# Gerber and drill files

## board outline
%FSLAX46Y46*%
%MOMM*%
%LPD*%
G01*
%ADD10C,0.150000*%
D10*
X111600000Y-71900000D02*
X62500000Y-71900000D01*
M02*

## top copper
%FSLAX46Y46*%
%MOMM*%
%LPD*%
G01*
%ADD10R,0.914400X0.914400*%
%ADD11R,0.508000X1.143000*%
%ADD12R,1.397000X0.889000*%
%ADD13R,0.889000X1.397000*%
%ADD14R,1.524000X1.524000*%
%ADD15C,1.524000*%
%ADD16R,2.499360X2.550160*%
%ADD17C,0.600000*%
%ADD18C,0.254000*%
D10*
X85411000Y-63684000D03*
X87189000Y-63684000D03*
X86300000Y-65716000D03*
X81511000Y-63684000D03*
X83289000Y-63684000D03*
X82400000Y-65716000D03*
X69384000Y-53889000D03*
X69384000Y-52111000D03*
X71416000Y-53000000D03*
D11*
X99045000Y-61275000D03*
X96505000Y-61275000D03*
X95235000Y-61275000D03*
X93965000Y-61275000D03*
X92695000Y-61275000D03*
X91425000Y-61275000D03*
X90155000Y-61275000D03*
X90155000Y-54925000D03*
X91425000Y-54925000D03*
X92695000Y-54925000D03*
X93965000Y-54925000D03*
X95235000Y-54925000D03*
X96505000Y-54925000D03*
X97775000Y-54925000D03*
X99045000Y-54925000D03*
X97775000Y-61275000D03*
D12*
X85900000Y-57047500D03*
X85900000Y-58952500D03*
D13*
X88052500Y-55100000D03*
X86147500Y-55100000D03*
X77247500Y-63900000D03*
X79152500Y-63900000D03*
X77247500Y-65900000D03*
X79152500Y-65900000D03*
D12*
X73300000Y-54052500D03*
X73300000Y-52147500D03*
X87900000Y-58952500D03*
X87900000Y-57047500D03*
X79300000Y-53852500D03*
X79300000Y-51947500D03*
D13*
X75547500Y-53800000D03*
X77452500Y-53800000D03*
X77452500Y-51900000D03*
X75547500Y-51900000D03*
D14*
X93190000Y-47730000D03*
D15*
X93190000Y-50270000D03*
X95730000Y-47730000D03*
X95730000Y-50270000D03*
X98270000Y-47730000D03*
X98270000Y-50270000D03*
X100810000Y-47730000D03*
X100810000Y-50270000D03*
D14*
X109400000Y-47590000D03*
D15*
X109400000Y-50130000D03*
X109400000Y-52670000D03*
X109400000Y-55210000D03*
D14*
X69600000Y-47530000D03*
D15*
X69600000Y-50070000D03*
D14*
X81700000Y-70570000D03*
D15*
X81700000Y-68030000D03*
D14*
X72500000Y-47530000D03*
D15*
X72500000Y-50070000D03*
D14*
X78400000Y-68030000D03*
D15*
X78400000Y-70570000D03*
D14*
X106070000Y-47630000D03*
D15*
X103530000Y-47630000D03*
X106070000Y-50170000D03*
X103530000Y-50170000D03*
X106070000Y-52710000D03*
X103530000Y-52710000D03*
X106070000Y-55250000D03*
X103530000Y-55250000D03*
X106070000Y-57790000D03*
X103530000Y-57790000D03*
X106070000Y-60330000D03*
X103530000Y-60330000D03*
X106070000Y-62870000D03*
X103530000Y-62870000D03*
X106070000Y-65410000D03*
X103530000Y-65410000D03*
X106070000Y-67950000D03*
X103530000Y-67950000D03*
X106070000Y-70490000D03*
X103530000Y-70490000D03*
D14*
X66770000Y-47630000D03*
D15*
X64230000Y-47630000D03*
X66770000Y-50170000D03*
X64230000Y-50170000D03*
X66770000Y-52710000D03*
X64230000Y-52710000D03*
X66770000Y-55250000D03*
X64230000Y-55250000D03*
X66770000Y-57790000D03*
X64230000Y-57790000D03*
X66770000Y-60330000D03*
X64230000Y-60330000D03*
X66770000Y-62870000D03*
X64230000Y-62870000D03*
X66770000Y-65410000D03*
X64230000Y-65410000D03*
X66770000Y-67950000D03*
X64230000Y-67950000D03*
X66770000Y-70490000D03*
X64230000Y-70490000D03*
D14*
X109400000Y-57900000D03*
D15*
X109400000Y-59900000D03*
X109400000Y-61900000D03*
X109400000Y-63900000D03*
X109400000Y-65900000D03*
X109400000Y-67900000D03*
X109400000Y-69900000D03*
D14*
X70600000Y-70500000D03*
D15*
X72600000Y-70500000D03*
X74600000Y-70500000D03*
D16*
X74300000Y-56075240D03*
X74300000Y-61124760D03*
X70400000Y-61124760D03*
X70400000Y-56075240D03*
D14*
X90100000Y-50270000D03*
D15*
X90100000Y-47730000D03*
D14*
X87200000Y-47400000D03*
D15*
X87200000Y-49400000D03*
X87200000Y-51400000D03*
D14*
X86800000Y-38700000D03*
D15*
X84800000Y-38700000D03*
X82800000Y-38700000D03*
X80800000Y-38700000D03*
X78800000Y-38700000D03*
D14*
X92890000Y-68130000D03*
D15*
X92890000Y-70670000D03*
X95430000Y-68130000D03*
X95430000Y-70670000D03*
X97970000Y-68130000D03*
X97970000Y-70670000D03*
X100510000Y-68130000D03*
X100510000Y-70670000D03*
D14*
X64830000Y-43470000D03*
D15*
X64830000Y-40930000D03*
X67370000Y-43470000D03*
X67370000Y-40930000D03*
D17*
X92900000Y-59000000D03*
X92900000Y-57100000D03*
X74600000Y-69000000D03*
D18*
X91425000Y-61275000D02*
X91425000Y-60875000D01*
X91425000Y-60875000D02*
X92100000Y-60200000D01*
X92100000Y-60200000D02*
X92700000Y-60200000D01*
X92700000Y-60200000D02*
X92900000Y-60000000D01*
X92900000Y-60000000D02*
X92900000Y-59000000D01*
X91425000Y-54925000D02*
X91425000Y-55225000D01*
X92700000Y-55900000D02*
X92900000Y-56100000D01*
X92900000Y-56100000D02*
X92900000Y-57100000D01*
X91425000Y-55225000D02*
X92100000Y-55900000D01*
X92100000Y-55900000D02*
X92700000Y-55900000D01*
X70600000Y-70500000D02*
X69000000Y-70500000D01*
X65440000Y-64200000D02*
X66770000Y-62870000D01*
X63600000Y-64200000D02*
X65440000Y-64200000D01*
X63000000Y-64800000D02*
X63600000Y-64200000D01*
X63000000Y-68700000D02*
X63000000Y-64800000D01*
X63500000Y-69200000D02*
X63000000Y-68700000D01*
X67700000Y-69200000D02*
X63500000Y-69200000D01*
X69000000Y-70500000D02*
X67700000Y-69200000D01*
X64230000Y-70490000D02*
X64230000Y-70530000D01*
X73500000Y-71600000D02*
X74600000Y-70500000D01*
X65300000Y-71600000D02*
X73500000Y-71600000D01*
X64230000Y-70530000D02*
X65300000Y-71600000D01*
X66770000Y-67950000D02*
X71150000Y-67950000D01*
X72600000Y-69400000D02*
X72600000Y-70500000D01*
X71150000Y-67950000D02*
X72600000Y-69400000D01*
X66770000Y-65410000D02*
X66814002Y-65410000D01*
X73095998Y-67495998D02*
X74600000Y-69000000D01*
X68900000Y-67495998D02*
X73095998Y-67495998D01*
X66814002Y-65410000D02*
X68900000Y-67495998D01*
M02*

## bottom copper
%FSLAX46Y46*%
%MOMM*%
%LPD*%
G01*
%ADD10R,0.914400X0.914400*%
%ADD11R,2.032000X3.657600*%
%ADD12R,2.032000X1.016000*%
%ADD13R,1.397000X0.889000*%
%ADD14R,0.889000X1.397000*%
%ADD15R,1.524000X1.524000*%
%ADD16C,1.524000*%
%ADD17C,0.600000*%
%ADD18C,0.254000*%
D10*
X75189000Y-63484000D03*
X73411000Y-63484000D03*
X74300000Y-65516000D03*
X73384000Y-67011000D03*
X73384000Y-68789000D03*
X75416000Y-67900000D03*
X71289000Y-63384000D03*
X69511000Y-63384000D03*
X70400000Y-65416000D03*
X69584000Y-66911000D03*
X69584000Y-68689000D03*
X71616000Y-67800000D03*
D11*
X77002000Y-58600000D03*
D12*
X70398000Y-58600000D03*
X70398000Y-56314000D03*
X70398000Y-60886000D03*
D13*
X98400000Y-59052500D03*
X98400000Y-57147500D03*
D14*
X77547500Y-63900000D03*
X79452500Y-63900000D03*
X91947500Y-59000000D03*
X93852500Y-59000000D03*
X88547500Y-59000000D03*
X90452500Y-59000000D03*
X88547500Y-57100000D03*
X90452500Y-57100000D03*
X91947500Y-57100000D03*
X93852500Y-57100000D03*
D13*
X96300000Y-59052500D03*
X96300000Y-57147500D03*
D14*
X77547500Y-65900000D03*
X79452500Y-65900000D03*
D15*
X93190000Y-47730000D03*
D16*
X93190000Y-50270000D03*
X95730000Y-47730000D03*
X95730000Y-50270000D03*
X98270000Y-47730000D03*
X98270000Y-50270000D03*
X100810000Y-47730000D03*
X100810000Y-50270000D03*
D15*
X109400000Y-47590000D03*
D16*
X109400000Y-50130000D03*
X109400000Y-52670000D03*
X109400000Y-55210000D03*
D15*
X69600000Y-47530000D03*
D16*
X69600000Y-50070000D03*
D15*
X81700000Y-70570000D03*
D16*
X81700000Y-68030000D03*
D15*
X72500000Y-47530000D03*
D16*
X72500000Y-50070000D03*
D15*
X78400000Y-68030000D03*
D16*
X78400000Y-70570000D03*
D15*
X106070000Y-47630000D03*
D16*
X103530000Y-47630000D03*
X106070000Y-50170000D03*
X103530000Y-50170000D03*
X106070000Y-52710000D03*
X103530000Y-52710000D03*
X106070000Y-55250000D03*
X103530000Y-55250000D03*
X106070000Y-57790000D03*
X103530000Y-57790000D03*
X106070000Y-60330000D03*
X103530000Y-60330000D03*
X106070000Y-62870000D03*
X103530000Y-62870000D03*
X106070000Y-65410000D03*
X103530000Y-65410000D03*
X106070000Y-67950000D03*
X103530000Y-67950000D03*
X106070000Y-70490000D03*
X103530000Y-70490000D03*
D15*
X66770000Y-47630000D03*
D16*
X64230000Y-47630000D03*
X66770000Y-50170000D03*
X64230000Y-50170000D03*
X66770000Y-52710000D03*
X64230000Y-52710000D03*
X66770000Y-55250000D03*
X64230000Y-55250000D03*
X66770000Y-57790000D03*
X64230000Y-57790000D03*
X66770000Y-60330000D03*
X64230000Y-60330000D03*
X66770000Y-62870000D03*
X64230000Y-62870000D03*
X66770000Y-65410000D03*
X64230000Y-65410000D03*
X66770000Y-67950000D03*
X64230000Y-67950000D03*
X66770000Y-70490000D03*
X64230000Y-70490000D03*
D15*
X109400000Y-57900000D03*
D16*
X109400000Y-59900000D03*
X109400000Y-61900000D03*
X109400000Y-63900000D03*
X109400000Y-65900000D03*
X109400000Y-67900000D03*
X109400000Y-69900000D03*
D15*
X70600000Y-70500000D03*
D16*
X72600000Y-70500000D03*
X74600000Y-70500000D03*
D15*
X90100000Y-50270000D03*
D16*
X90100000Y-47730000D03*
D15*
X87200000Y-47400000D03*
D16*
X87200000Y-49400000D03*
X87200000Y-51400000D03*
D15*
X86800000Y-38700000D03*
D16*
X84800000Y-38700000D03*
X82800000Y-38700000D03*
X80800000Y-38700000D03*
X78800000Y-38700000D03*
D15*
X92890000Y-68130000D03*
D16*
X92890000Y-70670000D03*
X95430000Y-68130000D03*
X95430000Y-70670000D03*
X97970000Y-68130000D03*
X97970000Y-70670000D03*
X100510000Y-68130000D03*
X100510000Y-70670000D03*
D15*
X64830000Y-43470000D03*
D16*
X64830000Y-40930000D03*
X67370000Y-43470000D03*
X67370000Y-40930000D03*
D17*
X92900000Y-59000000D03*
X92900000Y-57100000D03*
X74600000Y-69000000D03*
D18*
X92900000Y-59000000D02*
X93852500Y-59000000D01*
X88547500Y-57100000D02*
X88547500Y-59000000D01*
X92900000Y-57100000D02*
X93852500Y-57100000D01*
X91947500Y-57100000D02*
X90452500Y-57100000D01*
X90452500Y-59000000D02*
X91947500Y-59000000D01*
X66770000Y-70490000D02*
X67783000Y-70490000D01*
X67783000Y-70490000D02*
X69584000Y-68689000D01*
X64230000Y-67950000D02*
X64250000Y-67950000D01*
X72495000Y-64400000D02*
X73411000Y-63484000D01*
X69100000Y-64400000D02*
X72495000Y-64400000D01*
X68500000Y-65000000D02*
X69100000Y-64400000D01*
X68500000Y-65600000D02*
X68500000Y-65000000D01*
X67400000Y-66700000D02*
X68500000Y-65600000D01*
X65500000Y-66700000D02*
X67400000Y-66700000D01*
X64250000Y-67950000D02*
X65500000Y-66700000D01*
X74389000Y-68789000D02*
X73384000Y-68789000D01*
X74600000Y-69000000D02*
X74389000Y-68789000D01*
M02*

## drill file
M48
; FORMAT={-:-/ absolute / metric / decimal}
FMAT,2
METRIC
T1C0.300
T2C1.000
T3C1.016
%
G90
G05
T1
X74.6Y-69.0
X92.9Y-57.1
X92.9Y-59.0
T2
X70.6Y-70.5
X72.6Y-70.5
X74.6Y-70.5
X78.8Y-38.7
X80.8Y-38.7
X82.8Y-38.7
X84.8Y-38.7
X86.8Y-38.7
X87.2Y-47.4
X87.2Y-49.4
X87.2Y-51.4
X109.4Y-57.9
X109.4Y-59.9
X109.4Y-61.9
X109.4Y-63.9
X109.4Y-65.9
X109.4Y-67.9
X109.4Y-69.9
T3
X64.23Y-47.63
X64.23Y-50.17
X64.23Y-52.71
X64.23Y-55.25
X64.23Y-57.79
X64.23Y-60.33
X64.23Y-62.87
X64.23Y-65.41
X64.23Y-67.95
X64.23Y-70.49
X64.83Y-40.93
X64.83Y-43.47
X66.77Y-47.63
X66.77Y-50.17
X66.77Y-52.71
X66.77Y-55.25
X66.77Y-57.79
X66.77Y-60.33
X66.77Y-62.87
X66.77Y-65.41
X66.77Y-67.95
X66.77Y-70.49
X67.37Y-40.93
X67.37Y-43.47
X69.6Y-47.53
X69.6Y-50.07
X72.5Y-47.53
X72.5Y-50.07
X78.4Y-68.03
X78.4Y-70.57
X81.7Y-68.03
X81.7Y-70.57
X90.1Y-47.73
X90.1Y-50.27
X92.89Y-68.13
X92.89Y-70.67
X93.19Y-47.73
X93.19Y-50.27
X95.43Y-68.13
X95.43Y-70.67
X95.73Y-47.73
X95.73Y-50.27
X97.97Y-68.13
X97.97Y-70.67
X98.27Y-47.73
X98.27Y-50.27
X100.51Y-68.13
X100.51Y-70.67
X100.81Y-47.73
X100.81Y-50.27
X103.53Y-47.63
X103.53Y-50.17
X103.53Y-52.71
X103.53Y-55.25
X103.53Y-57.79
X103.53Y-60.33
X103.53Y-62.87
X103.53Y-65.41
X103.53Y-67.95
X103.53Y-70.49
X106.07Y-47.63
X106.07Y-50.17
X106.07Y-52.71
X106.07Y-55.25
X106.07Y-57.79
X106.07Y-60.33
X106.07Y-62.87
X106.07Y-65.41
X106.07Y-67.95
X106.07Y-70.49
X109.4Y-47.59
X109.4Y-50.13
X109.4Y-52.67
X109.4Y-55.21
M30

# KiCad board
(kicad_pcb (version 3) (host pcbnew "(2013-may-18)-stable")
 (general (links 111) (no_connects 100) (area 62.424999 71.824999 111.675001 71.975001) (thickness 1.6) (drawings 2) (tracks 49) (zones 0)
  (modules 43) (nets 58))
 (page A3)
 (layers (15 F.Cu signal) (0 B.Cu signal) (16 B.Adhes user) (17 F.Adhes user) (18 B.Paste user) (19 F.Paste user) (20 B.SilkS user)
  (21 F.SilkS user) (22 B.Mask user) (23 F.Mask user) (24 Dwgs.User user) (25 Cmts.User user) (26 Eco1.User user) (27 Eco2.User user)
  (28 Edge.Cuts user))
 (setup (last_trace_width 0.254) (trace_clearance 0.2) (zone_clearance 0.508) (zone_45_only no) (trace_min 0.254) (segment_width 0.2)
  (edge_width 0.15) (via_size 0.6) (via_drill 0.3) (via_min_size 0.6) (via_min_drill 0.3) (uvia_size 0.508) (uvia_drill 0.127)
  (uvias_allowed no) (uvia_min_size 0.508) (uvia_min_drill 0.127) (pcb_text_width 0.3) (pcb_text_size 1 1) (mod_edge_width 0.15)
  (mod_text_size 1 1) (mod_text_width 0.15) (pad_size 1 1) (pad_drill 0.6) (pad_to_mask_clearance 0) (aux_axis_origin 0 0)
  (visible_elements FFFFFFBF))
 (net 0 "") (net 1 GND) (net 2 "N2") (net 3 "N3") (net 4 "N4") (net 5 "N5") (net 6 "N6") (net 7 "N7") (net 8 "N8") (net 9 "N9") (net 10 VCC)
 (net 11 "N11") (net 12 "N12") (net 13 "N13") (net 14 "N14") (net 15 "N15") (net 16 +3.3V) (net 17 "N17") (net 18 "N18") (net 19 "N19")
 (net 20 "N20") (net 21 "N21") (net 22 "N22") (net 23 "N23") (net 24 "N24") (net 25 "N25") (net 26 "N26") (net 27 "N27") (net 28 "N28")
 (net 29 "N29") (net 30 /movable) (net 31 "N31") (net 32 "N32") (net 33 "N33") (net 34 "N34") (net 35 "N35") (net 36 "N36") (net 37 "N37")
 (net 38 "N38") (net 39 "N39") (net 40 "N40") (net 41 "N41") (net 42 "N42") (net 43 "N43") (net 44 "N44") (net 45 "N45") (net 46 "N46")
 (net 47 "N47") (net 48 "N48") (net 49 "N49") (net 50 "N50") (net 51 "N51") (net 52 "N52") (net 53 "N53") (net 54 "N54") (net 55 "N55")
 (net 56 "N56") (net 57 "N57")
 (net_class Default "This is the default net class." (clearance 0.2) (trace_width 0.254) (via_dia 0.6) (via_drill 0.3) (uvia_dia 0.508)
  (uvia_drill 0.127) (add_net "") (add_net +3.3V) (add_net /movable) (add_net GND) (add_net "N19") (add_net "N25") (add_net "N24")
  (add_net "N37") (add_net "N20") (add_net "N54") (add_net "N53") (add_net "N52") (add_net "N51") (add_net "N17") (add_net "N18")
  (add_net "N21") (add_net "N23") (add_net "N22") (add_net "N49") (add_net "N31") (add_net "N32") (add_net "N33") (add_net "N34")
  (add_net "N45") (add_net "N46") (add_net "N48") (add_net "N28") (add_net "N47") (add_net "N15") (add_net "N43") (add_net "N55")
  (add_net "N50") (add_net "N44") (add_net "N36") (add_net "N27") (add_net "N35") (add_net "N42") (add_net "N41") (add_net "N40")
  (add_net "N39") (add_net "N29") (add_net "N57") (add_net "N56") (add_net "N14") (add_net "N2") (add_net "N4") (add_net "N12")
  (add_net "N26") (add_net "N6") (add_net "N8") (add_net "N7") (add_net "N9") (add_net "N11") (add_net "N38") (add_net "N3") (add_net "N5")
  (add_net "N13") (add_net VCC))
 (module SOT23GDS (layer B.Cu) (at 74.3 64.5 180)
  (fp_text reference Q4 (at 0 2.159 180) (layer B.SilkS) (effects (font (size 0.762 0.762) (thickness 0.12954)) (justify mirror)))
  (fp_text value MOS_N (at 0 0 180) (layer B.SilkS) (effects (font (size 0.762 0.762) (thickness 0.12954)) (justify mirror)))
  (pad S smd rect (at -0.889 1.016 180) (size 0.9144 0.9144) (layers B.Cu B.Paste B.Mask) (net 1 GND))
  (pad G smd rect (at 0.889 1.016 180) (size 0.9144 0.9144) (layers B.Cu B.Paste B.Mask) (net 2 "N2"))
  (pad D smd rect (at 0 -1.016 180) (size 0.9144 0.9144) (layers B.Cu B.Paste B.Mask) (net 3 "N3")))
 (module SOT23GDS (layer B.Cu) (at 74.4 67.9 270)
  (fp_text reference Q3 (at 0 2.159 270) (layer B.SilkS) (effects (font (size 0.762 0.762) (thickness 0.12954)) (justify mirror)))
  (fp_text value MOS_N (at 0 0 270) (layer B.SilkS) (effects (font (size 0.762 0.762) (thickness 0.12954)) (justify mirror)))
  (pad S smd rect (at -0.889 1.016 270) (size 0.9144 0.9144) (layers B.Cu B.Paste B.Mask) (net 1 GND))
  (pad G smd rect (at 0.889 1.016 270) (size 0.9144 0.9144) (layers B.Cu B.Paste B.Mask) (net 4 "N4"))
  (pad D smd rect (at 0 -1.016 270) (size 0.9144 0.9144) (layers B.Cu B.Paste B.Mask) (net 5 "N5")))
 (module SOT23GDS (layer F.Cu) (at 86.3 64.7)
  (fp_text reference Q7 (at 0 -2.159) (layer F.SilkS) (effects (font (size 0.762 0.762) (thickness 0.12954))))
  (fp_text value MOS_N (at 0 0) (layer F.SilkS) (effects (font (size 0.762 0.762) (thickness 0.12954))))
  (pad S smd rect (at -0.889 -1.016) (size 0.9144 0.9144) (layers F.Cu F.Paste F.Mask) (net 1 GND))
  (pad G smd rect (at 0.889 -1.016) (size 0.9144 0.9144) (layers F.Cu F.Paste F.Mask) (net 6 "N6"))
  (pad D smd rect (at 0 1.016) (size 0.9144 0.9144) (layers F.Cu F.Paste F.Mask) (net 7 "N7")))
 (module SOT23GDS (layer F.Cu) (at 82.4 64.7)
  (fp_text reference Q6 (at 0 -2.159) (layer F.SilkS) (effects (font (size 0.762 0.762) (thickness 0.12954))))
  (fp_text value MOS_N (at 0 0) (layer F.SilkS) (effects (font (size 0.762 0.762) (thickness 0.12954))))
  (pad S smd rect (at -0.889 -1.016) (size 0.9144 0.9144) (layers F.Cu F.Paste F.Mask) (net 1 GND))
  (pad G smd rect (at 0.889 -1.016) (size 0.9144 0.9144) (layers F.Cu F.Paste F.Mask) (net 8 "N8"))
  (pad D smd rect (at 0 1.016) (size 0.9144 0.9144) (layers F.Cu F.Paste F.Mask) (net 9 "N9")))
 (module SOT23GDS (layer F.Cu) (at 70.4 53 90)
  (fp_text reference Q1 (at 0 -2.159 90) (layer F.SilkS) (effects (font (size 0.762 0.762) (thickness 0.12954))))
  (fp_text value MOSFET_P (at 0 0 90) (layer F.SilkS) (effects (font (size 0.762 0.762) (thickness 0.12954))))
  (pad S smd rect (at -0.889 -1.016 90) (size 0.9144 0.9144) (layers F.Cu F.Paste F.Mask) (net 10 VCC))
  (pad G smd rect (at 0.889 -1.016 90) (size 0.9144 0.9144) (layers F.Cu F.Paste F.Mask) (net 1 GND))
  (pad D smd rect (at 0 1.016 90) (size 0.9144 0.9144) (layers F.Cu F.Paste F.Mask) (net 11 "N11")))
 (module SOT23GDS (layer B.Cu) (at 70.4 64.4 180)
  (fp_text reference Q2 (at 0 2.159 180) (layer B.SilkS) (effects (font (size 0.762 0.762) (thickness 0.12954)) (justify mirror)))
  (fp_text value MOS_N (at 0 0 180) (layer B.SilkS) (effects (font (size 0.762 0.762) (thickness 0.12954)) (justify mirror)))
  (pad S smd rect (at -0.889 1.016 180) (size 0.9144 0.9144) (layers B.Cu B.Paste B.Mask) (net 1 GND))
  (pad G smd rect (at 0.889 1.016 180) (size 0.9144 0.9144) (layers B.Cu B.Paste B.Mask) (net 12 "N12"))
  (pad D smd rect (at 0 -1.016 180) (size 0.9144 0.9144) (layers B.Cu B.Paste B.Mask) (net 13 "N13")))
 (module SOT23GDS (layer B.Cu) (at 70.6 67.8 270)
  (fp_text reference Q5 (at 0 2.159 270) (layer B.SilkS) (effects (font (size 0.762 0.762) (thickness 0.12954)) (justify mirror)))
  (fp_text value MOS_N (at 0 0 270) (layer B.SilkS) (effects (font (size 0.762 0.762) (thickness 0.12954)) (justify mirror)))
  (pad S smd rect (at -0.889 1.016 270) (size 0.9144 0.9144) (layers B.Cu B.Paste B.Mask) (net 1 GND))
  (pad G smd rect (at 0.889 1.016 270) (size 0.9144 0.9144) (layers B.Cu B.Paste B.Mask) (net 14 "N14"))
  (pad D smd rect (at 0 -1.016 270) (size 0.9144 0.9144) (layers B.Cu B.Paste B.Mask) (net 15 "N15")))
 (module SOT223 (layer B.Cu) (at 73.7 58.6 90)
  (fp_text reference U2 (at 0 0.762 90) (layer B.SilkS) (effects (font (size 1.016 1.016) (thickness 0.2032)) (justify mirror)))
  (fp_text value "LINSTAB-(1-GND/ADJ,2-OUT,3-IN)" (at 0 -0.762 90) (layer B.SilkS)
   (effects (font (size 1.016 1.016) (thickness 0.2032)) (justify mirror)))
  (pad 4 smd rect (at 0 3.302 90) (size 3.6576 2.032) (layers B.Cu B.Paste B.Mask))
  (pad 2 smd rect (at 0 -3.302 90) (size 1.016 2.032) (layers B.Cu B.Paste B.Mask) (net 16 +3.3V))
  (pad 3 smd rect (at 2.286 -3.302 90) (size 1.016 2.032) (layers B.Cu B.Paste B.Mask) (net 10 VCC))
  (pad 1 smd rect (at -2.286 -3.302 90) (size 1.016 2.032) (layers B.Cu B.Paste B.Mask) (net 1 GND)))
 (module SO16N (layer F.Cu) (at 94.6 58.1 180)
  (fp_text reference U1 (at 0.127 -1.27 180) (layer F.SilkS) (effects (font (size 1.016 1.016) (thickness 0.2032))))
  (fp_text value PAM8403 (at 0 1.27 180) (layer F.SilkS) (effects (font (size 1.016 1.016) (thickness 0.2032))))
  (pad 16 smd rect (at -4.445 -3.175 180) (size 0.508 1.143) (layers F.Cu F.Paste F.Mask) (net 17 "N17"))
  (pad 14 smd rect (at -1.905 -3.175 180) (size 0.508 1.143) (layers F.Cu F.Paste F.Mask) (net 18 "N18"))
  (pad 13 smd rect (at -0.635 -3.175 180) (size 0.508 1.143) (layers F.Cu F.Paste F.Mask) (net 10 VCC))
  (pad 12 smd rect (at 0.635 -3.175 180) (size 0.508 1.143) (layers F.Cu F.Paste F.Mask) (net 10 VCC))
  (pad 11 smd rect (at 1.905 -3.175 180) (size 0.508 1.143) (layers F.Cu F.Paste F.Mask) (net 1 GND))
  (pad 10 smd rect (at 3.175 -3.175 180) (size 0.508 1.143) (layers F.Cu F.Paste F.Mask) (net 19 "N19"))
  (pad 9 smd rect (at 4.445 -3.175 180) (size 0.508 1.143) (layers F.Cu F.Paste F.Mask) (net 1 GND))
  (pad 8 smd rect (at 4.445 3.175 180) (size 0.508 1.143) (layers F.Cu F.Paste F.Mask) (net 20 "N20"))
  (pad 7 smd rect (at 3.175 3.175 180) (size 0.508 1.143) (layers F.Cu F.Paste F.Mask) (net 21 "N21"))
  (pad 6 smd rect (at 1.905 3.175 180) (size 0.508 1.143) (layers F.Cu F.Paste F.Mask) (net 10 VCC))
  (pad 5 smd rect (at 0.635 3.175 180) (size 0.508 1.143) (layers F.Cu F.Paste F.Mask) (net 10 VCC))
  (pad 4 smd rect (at -0.635 3.175 180) (size 0.508 1.143) (layers F.Cu F.Paste F.Mask) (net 10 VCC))
  (pad 3 smd rect (at -1.905 3.175 180) (size 0.508 1.143) (layers F.Cu F.Paste F.Mask) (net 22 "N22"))
  (pad 2 smd rect (at -3.175 3.175 180) (size 0.508 1.143) (layers F.Cu F.Paste F.Mask) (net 1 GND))
  (pad 1 smd rect (at -4.445 3.175 180) (size 0.508 1.143) (layers F.Cu F.Paste F.Mask) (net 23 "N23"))
  (pad 15 smd rect (at -3.175 -3.175 180) (size 0.508 1.143) (layers F.Cu F.Paste F.Mask) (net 1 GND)))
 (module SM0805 (layer B.Cu) (at 98.4 58.1 90)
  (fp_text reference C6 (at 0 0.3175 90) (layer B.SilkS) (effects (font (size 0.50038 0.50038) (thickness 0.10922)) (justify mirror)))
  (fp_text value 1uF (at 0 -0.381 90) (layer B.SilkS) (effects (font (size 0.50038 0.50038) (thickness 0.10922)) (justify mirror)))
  (pad 1 smd rect (at -0.9525 0 90) (size 0.889 1.397) (layers B.Cu B.Paste B.Mask) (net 10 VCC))
  (pad 2 smd rect (at 0.9525 0 90) (size 0.889 1.397) (layers B.Cu B.Paste B.Mask) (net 1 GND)))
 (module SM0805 (layer F.Cu) (at 85.9 58 270)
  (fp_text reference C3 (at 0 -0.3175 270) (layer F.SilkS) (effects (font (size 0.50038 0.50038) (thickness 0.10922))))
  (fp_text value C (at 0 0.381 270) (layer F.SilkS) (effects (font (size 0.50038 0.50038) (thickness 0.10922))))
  (pad 1 smd rect (at -0.9525 0 270) (size 0.889 1.397) (layers F.Cu F.Paste F.Mask) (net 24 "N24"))
  (pad 2 smd rect (at 0.9525 0 270) (size 0.889 1.397) (layers F.Cu F.Paste F.Mask) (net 1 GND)))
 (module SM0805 (layer F.Cu) (at 87.1 55.1 180)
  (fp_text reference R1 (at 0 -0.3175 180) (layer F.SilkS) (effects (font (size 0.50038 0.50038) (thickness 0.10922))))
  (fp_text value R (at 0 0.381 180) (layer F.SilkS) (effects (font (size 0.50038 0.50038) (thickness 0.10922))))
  (pad 1 smd rect (at -0.9525 0 180) (size 0.889 1.397) (layers F.Cu F.Paste F.Mask) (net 24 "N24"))
  (pad 2 smd rect (at 0.9525 0 180) (size 0.889 1.397) (layers F.Cu F.Paste F.Mask) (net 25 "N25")))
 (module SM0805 (layer F.Cu) (at 78.2 63.9)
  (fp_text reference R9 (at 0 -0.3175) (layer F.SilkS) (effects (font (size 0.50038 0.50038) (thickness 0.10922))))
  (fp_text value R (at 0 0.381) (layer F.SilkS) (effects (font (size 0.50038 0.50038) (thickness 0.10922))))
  (pad 1 smd rect (at -0.9525 0) (size 0.889 1.397) (layers F.Cu F.Paste F.Mask) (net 15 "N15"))
  (pad 2 smd rect (at 0.9525 0) (size 0.889 1.397) (layers F.Cu F.Paste F.Mask) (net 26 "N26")))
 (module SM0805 (layer B.Cu) (at 78.5 63.9)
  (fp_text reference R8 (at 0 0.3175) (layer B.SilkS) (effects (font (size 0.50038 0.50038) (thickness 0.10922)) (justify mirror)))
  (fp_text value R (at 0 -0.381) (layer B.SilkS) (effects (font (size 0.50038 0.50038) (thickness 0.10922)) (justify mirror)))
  (pad 1 smd rect (at -0.9525 0) (size 0.889 1.397) (layers B.Cu B.Paste B.Mask) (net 3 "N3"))
  (pad 2 smd rect (at 0.9525 0) (size 0.889 1.397) (layers B.Cu B.Paste B.Mask) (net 26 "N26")))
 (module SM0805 (layer F.Cu) (at 78.2 65.9)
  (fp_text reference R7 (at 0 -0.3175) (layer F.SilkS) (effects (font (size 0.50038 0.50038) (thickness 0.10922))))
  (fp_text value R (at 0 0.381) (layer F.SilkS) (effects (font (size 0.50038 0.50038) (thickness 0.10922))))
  (pad 1 smd rect (at -0.9525 0) (size 0.889 1.397) (layers F.Cu F.Paste F.Mask) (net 5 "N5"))
  (pad 2 smd rect (at 0.9525 0) (size 0.889 1.397) (layers F.Cu F.Paste F.Mask) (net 26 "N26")))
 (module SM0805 (layer B.Cu) (at 92.9 59)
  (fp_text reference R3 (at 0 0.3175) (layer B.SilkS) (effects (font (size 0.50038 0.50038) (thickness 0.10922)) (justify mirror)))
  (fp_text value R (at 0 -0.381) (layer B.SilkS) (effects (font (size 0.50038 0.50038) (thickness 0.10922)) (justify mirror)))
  (pad 1 smd rect (at -0.9525 0) (size 0.889 1.397) (layers B.Cu B.Paste B.Mask) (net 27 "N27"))
  (pad 2 smd rect (at 0.9525 0) (size 0.889 1.397) (layers B.Cu B.Paste B.Mask) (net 19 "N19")))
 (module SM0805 (layer B.Cu) (at 89.5 59)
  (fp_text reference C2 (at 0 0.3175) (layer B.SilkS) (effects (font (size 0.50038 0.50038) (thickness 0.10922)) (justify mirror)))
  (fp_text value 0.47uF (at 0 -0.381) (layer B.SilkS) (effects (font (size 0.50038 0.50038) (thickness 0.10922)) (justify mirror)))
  (pad 1 smd rect (at -0.9525 0) (size 0.889 1.397) (layers B.Cu B.Paste B.Mask) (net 24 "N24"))
  (pad 2 smd rect (at 0.9525 0) (size 0.889 1.397) (layers B.Cu B.Paste B.Mask) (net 27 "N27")))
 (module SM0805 (layer B.Cu) (at 89.5 57.1)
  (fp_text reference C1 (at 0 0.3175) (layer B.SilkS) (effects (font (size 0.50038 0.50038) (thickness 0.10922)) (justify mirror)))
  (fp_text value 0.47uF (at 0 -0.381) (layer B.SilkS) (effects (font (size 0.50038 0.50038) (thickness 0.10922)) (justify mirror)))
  (pad 1 smd rect (at -0.9525 0) (size 0.889 1.397) (layers B.Cu B.Paste B.Mask) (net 24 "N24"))
  (pad 2 smd rect (at 0.9525 0) (size 0.889 1.397) (layers B.Cu B.Paste B.Mask) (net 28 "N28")))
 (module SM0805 (layer B.Cu) (at 92.9 57.1)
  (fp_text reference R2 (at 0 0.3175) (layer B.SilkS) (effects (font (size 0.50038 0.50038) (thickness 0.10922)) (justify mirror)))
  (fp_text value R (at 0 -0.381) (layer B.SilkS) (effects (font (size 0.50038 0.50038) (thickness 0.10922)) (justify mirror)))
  (pad 1 smd rect (at -0.9525 0) (size 0.889 1.397) (layers B.Cu B.Paste B.Mask) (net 28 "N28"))
  (pad 2 smd rect (at 0.9525 0) (size 0.889 1.397) (layers B.Cu B.Paste B.Mask) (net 21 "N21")))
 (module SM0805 (layer F.Cu) (at 73.3 53.1 90)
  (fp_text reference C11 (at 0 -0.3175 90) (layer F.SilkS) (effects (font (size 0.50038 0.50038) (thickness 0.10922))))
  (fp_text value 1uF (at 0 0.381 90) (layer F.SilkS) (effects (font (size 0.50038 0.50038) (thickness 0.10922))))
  (pad 1 smd rect (at -0.9525 0 90) (size 0.889 1.397) (layers F.Cu F.Paste F.Mask) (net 10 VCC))
  (pad 2 smd rect (at 0.9525 0 90) (size 0.889 1.397) (layers F.Cu F.Paste F.Mask) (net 1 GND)))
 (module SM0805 (layer B.Cu) (at 96.3 58.1 90)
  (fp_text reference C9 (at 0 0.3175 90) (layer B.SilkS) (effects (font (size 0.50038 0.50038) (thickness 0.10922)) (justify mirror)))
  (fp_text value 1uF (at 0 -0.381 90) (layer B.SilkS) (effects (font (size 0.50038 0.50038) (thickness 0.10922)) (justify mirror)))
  (pad 1 smd rect (at -0.9525 0 90) (size 0.889 1.397) (layers B.Cu B.Paste B.Mask) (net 10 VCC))
  (pad 2 smd rect (at 0.9525 0 90) (size 0.889 1.397) (layers B.Cu B.Paste B.Mask) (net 1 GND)))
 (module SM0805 (layer B.Cu) (at 78.5 65.9)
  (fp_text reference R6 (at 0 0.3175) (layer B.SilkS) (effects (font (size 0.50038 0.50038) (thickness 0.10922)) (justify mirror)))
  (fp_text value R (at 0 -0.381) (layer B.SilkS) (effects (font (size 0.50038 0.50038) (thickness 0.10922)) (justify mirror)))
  (pad 1 smd rect (at -0.9525 0) (size 0.889 1.397) (layers B.Cu B.Paste B.Mask) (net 13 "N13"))
  (pad 2 smd rect (at 0.9525 0) (size 0.889 1.397) (layers B.Cu B.Paste B.Mask) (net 26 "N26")))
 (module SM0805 (layer F.Cu) (at 87.9 58 90)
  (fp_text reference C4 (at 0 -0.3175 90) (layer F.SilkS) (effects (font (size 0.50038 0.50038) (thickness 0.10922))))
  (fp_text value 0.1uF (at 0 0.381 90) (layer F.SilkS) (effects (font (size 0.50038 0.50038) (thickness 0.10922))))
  (pad 1 smd rect (at -0.9525 0 90) (size 0.889 1.397) (layers F.Cu F.Paste F.Mask) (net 1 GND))
  (pad 2 smd rect (at 0.9525 0 90) (size 0.889 1.397) (layers F.Cu F.Paste F.Mask) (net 20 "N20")))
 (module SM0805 (layer F.Cu) (at 79.3 52.9 90)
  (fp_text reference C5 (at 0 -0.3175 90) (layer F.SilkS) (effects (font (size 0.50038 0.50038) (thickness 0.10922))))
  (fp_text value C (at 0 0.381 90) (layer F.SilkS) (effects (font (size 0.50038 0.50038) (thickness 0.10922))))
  (pad 1 smd rect (at -0.9525 0 90) (size 0.889 1.397) (layers F.Cu F.Paste F.Mask) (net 10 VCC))
  (pad 2 smd rect (at 0.9525 0 90) (size 0.889 1.397) (layers F.Cu F.Paste F.Mask) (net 1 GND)))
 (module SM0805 (layer F.Cu) (at 76.5 53.8)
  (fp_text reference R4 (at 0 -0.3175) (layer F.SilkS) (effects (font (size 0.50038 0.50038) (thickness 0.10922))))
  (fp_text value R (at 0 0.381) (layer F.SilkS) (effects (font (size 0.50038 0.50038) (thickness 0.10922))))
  (pad 1 smd rect (at -0.9525 0) (size 0.889 1.397) (layers F.Cu F.Paste F.Mask) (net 10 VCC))
  (pad 2 smd rect (at 0.9525 0) (size 0.889 1.397) (layers F.Cu F.Paste F.Mask) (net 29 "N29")))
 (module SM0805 (layer F.Cu) (at 76.5 51.9 180)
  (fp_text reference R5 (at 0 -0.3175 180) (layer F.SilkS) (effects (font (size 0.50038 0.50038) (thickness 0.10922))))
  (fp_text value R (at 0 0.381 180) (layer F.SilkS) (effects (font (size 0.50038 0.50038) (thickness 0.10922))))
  (pad 1 smd rect (at -0.9525 0 180) (size 0.889 1.397) (layers F.Cu F.Paste F.Mask) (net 29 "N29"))
  (pad 2 smd rect (at 0.9525 0 180) (size 0.889 1.397) (layers F.Cu F.Paste F.Mask) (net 1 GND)))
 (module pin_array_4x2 (layer B.Cu) (at 97 49)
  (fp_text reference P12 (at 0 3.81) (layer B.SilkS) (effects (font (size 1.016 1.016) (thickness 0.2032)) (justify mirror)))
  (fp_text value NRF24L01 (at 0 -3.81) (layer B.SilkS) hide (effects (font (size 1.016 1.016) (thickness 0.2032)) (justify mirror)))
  (pad 1 thru_hole rect (at -3.81 -1.27) (size 1.524 1.524) (drill 1.016) (layers *.Cu *.Mask B.SilkS) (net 1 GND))
  (pad 2 thru_hole circle (at -3.81 1.27) (size 1.524 1.524) (drill 1.016) (layers *.Cu *.Mask B.SilkS) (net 16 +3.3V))
  (pad 3 thru_hole circle (at -1.27 -1.27) (size 1.524 1.524) (drill 1.016) (layers *.Cu *.Mask B.SilkS) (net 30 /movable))
  (pad 4 thru_hole circle (at -1.27 1.27) (size 1.524 1.524) (drill 1.016) (layers *.Cu *.Mask B.SilkS) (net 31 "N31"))
  (pad 5 thru_hole circle (at 1.27 -1.27) (size 1.524 1.524) (drill 1.016) (layers *.Cu *.Mask B.SilkS) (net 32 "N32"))
  (pad 6 thru_hole circle (at 1.27 1.27) (size 1.524 1.524) (drill 1.016) (layers *.Cu *.Mask B.SilkS) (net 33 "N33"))
  (pad 7 thru_hole circle (at 3.81 -1.27) (size 1.524 1.524) (drill 1.016) (layers *.Cu *.Mask B.SilkS) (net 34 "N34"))
  (pad 8 thru_hole circle (at 3.81 1.27) (size 1.524 1.524) (drill 1.016) (layers *.Cu *.Mask B.SilkS) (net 30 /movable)))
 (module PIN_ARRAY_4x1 (layer B.Cu) (at 109.4 51.4 270)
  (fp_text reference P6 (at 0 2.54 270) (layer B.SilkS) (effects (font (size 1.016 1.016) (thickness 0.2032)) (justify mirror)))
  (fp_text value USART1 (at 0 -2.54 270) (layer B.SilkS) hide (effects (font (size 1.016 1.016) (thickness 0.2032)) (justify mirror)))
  (pad 1 thru_hole rect (at -3.81 0 270) (size 1.524 1.524) (drill 1.016) (layers *.Cu *.Mask B.SilkS) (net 1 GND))
  (pad 2 thru_hole circle (at -1.27 0 270) (size 1.524 1.524) (drill 1.016) (layers *.Cu *.Mask B.SilkS))
  (pad 3 thru_hole circle (at 1.27 0 270) (size 1.524 1.524) (drill 1.016) (layers *.Cu *.Mask B.SilkS) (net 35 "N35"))
  (pad 4 thru_hole circle (at 3.81 0 270) (size 1.524 1.524) (drill 1.016) (layers *.Cu *.Mask B.SilkS) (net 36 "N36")))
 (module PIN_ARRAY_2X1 (layer B.Cu) (at 69.6 48.8 270)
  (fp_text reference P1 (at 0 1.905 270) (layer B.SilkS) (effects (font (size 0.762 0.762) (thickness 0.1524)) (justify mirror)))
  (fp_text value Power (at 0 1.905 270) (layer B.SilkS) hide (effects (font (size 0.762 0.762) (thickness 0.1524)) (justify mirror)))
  (pad 1 thru_hole rect (at -1.27 0 270) (size 1.524 1.524) (drill 1.016) (layers *.Cu *.Mask B.SilkS) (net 1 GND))
  (pad 2 thru_hole circle (at 1.27 0 270) (size 1.524 1.524) (drill 1.016) (layers *.Cu *.Mask B.SilkS) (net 11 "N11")))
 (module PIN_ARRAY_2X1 (layer B.Cu) (at 81.7 69.3 90)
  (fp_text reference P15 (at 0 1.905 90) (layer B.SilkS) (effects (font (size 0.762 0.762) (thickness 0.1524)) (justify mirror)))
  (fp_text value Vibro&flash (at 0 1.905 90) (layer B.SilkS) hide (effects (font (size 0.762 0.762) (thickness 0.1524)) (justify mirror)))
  (pad 1 thru_hole rect (at -1.27 0 90) (size 1.524 1.524) (drill 1.016) (layers *.Cu *.Mask B.SilkS) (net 7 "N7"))
  (pad 2 thru_hole circle (at 1.27 0 90) (size 1.524 1.524) (drill 1.016) (layers *.Cu *.Mask B.SilkS) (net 9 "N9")))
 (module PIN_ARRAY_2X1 (layer B.Cu) (at 72.5 48.8 270)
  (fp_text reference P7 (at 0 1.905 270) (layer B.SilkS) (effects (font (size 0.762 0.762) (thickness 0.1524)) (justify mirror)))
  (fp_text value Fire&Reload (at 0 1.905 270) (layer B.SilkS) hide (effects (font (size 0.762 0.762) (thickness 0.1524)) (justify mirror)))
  (pad 1 thru_hole rect (at -1.27 0 270) (size 1.524 1.524) (drill 1.016) (layers *.Cu *.Mask B.SilkS) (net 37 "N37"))
  (pad 2 thru_hole circle (at 1.27 0 270) (size 1.524 1.524) (drill 1.016) (layers *.Cu *.Mask B.SilkS) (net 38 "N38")))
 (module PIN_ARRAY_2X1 (layer B.Cu) (at 78.4 69.3 270)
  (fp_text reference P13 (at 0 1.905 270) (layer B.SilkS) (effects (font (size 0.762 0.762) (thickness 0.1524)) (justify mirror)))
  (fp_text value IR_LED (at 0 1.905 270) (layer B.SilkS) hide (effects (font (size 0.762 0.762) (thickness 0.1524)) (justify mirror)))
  (pad 1 thru_hole rect (at -1.27 0 270) (size 1.524 1.524) (drill 1.016) (layers *.Cu *.Mask B.SilkS) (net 26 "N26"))
  (pad 2 thru_hole circle (at 1.27 0 270) (size 1.524 1.524) (drill 1.016) (layers *.Cu *.Mask B.SilkS) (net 10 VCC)))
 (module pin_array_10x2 (layer B.Cu) (at 104.8 59.1 270)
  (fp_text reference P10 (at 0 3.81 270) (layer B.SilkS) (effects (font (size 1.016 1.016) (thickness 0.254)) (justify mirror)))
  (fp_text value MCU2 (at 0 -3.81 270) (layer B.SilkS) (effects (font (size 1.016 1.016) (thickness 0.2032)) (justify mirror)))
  (pad 1 thru_hole rect (at -11.47 -1.27 270) (size 1.524 1.524) (drill 1.016) (layers *.Cu *.Mask B.SilkS) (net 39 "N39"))
  (pad 2 thru_hole circle (at -11.47 1.27 270) (size 1.524 1.524) (drill 1.016) (layers *.Cu *.Mask B.SilkS) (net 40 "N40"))
  (pad 3 thru_hole circle (at -8.93 -1.27 270) (size 1.524 1.524) (drill 1.016) (layers *.Cu *.Mask B.SilkS) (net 31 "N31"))
  (pad 4 thru_hole circle (at -8.93 1.27 270) (size 1.524 1.524) (drill 1.016) (layers *.Cu *.Mask B.SilkS) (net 32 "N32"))
  (pad 5 thru_hole circle (at -6.39 -1.27 270) (size 1.524 1.524) (drill 1.016) (layers *.Cu *.Mask B.SilkS) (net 34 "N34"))
  (pad 6 thru_hole circle (at -6.39 1.27 270) (size 1.524 1.524) (drill 1.016) (layers *.Cu *.Mask B.SilkS) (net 33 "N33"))
  (pad 7 thru_hole circle (at -3.85 -1.27 270) (size 1.524 1.524) (drill 1.016) (layers *.Cu *.Mask B.SilkS) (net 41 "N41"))
  (pad 8 thru_hole circle (at -3.85 1.27 270) (size 1.524 1.524) (drill 1.016) (layers *.Cu *.Mask B.SilkS) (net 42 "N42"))
  (pad 9 thru_hole circle (at -1.31 -1.27 270) (size 1.524 1.524) (drill 1.016) (layers *.Cu *.Mask B.SilkS) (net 35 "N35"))
  (pad 10 thru_hole circle (at -1.31 1.27 270) (size 1.524 1.524) (drill 1.016) (layers *.Cu *.Mask B.SilkS) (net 36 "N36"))
  (pad 11 thru_hole circle (at 1.23 -1.27 270) (size 1.524 1.524) (drill 1.016) (layers *.Cu *.Mask B.SilkS) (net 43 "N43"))
  (pad 12 thru_hole circle (at 1.23 1.27 270) (size 1.524 1.524) (drill 1.016) (layers *.Cu *.Mask B.SilkS) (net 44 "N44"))
  (pad 13 thru_hole circle (at 3.77 -1.27 270) (size 1.524 1.524) (drill 1.016) (layers *.Cu *.Mask B.SilkS) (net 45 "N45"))
  (pad 14 thru_hole circle (at 3.77 1.27 270) (size 1.524 1.524) (drill 1.016) (layers *.Cu *.Mask B.SilkS) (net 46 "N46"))
  (pad 15 thru_hole circle (at 6.31 -1.27 270) (size 1.524 1.524) (drill 1.016) (layers *.Cu *.Mask B.SilkS) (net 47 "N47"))
  (pad 16 thru_hole circle (at 6.31 1.27 270) (size 1.524 1.524) (drill 1.016) (layers *.Cu *.Mask B.SilkS) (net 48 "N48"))
  (pad 17 thru_hole circle (at 8.85 -1.27 270) (size 1.524 1.524) (drill 1.016) (layers *.Cu *.Mask B.SilkS) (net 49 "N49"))
  (pad 18 thru_hole circle (at 8.85 1.27 270) (size 1.524 1.524) (drill 1.016) (layers *.Cu *.Mask B.SilkS) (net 30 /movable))
  (pad 19 thru_hole circle (at 11.39 -1.27 270) (size 1.524 1.524) (drill 1.016) (layers *.Cu *.Mask B.SilkS) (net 30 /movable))
  (pad 20 thru_hole circle (at 11.39 1.27 270) (size 1.524 1.524) (drill 1.016) (layers *.Cu *.Mask B.SilkS) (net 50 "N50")))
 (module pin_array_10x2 (layer B.Cu) (at 65.5 59.1 270)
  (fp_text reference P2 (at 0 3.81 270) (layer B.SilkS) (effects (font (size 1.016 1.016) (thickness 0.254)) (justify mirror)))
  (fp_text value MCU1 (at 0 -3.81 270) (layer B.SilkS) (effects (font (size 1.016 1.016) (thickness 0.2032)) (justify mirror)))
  (pad 1 thru_hole rect (at -11.47 -1.27 270) (size 1.524 1.524) (drill 1.016) (layers *.Cu *.Mask B.SilkS) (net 1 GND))
  (pad 2 thru_hole circle (at -11.47 1.27 270) (size 1.524 1.524) (drill 1.016) (layers *.Cu *.Mask B.SilkS) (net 16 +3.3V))
  (pad 3 thru_hole circle (at -8.93 -1.27 270) (size 1.524 1.524) (drill 1.016) (layers *.Cu *.Mask B.SilkS))
  (pad 4 thru_hole circle (at -8.93 1.27 270) (size 1.524 1.524) (drill 1.016) (layers *.Cu *.Mask B.SilkS) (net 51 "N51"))
  (pad 5 thru_hole circle (at -6.39 -1.27 270) (size 1.524 1.524) (drill 1.016) (layers *.Cu *.Mask B.SilkS) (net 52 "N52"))
  (pad 6 thru_hole circle (at -6.39 1.27 270) (size 1.524 1.524) (drill 1.016) (layers *.Cu *.Mask B.SilkS) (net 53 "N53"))
  (pad 7 thru_hole circle (at -3.85 -1.27 270) (size 1.524 1.524) (drill 1.016) (layers *.Cu *.Mask B.SilkS) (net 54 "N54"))
  (pad 8 thru_hole circle (at -3.85 1.27 270) (size 1.524 1.524) (drill 1.016) (layers *.Cu *.Mask B.SilkS) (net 37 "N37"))
  (pad 9 thru_hole circle (at -1.31 -1.27 270) (size 1.524 1.524) (drill 1.016) (layers *.Cu *.Mask B.SilkS) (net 38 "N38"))
  (pad 10 thru_hole circle (at -1.31 1.27 270) (size 1.524 1.524) (drill 1.016) (layers *.Cu *.Mask B.SilkS) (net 8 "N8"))
  (pad 11 thru_hole circle (at 1.23 -1.27 270) (size 1.524 1.524) (drill 1.016) (layers *.Cu *.Mask B.SilkS) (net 6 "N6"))
  (pad 12 thru_hole circle (at 1.23 1.27 270) (size 1.524 1.524) (drill 1.016) (layers *.Cu *.Mask B.SilkS) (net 25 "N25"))
  (pad 13 thru_hole circle (at 3.77 -1.27 270) (size 1.524 1.524) (drill 1.016) (layers *.Cu *.Mask B.SilkS) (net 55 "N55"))
  (pad 14 thru_hole circle (at 3.77 1.27 270) (size 1.524 1.524) (drill 1.016) (layers *.Cu *.Mask B.SilkS) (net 12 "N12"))
  (pad 15 thru_hole circle (at 6.31 -1.27 270) (size 1.524 1.524) (drill 1.016) (layers *.Cu *.Mask B.SilkS) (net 4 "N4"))
  (pad 16 thru_hole circle (at 6.31 1.27 270) (size 1.524 1.524) (drill 1.016) (layers *.Cu *.Mask B.SilkS) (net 29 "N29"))
  (pad 17 thru_hole circle (at 8.85 -1.27 270) (size 1.524 1.524) (drill 1.016) (layers *.Cu *.Mask B.SilkS) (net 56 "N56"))
  (pad 18 thru_hole circle (at 8.85 1.27 270) (size 1.524 1.524) (drill 1.016) (layers *.Cu *.Mask B.SilkS) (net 2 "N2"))
  (pad 19 thru_hole circle (at 11.39 -1.27 270) (size 1.524 1.524) (drill 1.016) (layers *.Cu *.Mask B.SilkS) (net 14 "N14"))
  (pad 20 thru_hole circle (at 11.39 1.27 270) (size 1.524 1.524) (drill 1.016) (layers *.Cu *.Mask B.SilkS) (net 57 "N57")))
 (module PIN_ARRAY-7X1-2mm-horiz (layer F.Cu) (at 109.4 63.9 270)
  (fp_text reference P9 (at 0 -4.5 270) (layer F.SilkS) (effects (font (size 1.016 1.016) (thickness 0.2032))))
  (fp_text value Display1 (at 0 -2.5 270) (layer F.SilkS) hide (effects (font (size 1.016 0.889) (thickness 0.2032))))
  (pad 1 thru_hole rect (at -6 0 270) (size 1.524 1.524) (drill 1) (layers *.Cu *.Mask F.SilkS) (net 39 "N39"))
  (pad 2 thru_hole circle (at -4 0 270) (size 1.524 1.524) (drill 1) (layers *.Cu *.Mask F.SilkS) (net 40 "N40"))
  (pad 3 thru_hole circle (at -2 0 270) (size 1.524 1.524) (drill 1) (layers *.Cu *.Mask F.SilkS) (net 41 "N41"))
  (pad 4 thru_hole circle (at 0 0 270) (size 1.524 1.524) (drill 1) (layers *.Cu *.Mask F.SilkS) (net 42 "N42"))
  (pad 5 thru_hole circle (at 2 0 270) (size 1.524 1.524) (drill 1) (layers *.Cu *.Mask F.SilkS) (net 43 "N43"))
  (pad 6 thru_hole circle (at 4 0 270) (size 1.524 1.524) (drill 1) (layers *.Cu *.Mask F.SilkS) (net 44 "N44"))
  (pad 7 thru_hole circle (at 6 0 270) (size 1.524 1.524) (drill 1) (layers *.Cu *.Mask F.SilkS) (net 50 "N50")))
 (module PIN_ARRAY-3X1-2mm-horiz (layer B.Cu) (at 72.6 70.5)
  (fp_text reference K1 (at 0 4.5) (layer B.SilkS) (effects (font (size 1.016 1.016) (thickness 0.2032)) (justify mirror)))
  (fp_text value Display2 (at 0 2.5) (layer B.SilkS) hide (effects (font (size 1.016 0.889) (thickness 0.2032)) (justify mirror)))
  (pad 1 thru_hole rect (at -2 0) (size 1.524 1.524) (drill 1) (layers *.Cu *.Mask B.SilkS) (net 55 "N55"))
  (pad 2 thru_hole circle (at 0 0) (size 1.524 1.524) (drill 1) (layers *.Cu *.Mask B.SilkS) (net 56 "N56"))
  (pad 3 thru_hole circle (at 2 0) (size 1.524 1.524) (drill 1) (layers *.Cu *.Mask B.SilkS) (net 57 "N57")))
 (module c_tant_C (layer F.Cu) (at 74.3 58.6 90)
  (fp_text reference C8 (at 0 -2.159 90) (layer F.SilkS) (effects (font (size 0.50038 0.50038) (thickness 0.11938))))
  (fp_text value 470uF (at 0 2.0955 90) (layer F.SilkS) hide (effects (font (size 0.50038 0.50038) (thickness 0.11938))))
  (pad 1 smd rect (at 2.52476 0 90) (size 2.55016 2.49936) (layers F.Cu F.Paste F.Mask) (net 10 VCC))
  (pad 2 smd rect (at -2.52476 0 90) (size 2.55016 2.49936) (layers F.Cu F.Paste F.Mask) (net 1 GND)))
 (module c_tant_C (layer F.Cu) (at 70.4 58.6 270)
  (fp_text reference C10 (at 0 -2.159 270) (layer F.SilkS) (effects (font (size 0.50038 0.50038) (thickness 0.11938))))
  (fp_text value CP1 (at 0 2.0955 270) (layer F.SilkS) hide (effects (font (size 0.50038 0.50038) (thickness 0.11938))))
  (pad 1 smd rect (at 2.52476 0 270) (size 2.55016 2.49936) (layers F.Cu F.Paste F.Mask) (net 16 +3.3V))
  (pad 2 smd rect (at -2.52476 0 270) (size 2.55016 2.49936) (layers F.Cu F.Paste F.Mask) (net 1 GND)))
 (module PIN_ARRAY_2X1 (layer B.Cu) (at 90.1 49 90)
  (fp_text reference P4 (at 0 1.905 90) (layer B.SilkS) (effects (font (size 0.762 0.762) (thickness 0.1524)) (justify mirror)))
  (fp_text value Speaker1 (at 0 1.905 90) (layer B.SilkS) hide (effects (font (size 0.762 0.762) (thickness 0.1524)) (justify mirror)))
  (pad 1 thru_hole rect (at -1.27 0 90) (size 1.524 1.524) (drill 1.016) (layers *.Cu *.Mask B.SilkS) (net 22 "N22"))
  (pad 2 thru_hole circle (at 1.27 0 90) (size 1.524 1.524) (drill 1.016) (layers *.Cu *.Mask B.SilkS) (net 23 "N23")))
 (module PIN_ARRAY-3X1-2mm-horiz (layer B.Cu) (at 87.2 49.4 270)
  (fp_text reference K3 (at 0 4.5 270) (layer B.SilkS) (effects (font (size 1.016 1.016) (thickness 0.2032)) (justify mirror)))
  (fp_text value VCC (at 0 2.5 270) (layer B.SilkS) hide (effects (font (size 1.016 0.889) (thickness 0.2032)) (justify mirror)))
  (pad 1 thru_hole rect (at -2 0 270) (size 1.524 1.524) (drill 1) (layers *.Cu *.Mask B.SilkS) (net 10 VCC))
  (pad 2 thru_hole circle (at 0 0 270) (size 1.524 1.524) (drill 1) (layers *.Cu *.Mask B.SilkS) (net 10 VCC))
  (pad 3 thru_hole circle (at 2 0 270) (size 1.524 1.524) (drill 1) (layers *.Cu *.Mask B.SilkS) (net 10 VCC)))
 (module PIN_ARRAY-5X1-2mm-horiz (layer B.Cu) (at 82.8 38.7 180)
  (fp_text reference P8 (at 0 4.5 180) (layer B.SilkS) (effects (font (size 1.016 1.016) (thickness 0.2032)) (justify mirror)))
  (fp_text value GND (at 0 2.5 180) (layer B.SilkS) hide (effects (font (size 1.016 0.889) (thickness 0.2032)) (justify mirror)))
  (pad 1 thru_hole rect (at -4 0 180) (size 1.524 1.524) (drill 1) (layers *.Cu *.Mask B.SilkS) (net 1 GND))
  (pad 2 thru_hole circle (at -2 0 180) (size 1.524 1.524) (drill 1) (layers *.Cu *.Mask B.SilkS) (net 1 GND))
  (pad 3 thru_hole circle (at 0 0 180) (size 1.524 1.524) (drill 1) (layers *.Cu *.Mask B.SilkS) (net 1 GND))
  (pad 4 thru_hole circle (at 2 0 180) (size 1.524 1.524) (drill 1) (layers *.Cu *.Mask B.SilkS) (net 1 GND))
  (pad 5 thru_hole circle (at 4 0 180) (size 1.524 1.524) (drill 1) (layers *.Cu *.Mask B.SilkS) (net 1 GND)))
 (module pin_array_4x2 (layer B.Cu) (at 96.7 69.4)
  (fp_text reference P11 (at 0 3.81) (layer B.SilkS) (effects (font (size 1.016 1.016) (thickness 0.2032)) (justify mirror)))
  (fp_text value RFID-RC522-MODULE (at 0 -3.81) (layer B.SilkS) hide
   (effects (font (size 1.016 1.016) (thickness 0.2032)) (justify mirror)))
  (pad 1 thru_hole rect (at -3.81 -1.27) (size 1.524 1.524) (drill 1.016) (layers *.Cu *.Mask B.SilkS) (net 45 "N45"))
  (pad 2 thru_hole circle (at -3.81 1.27) (size 1.524 1.524) (drill 1.016) (layers *.Cu *.Mask B.SilkS) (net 46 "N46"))
  (pad 3 thru_hole circle (at -1.27 -1.27) (size 1.524 1.524) (drill 1.016) (layers *.Cu *.Mask B.SilkS) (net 48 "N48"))
  (pad 4 thru_hole circle (at -1.27 1.27) (size 1.524 1.524) (drill 1.016) (layers *.Cu *.Mask B.SilkS) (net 47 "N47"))
  (pad 5 thru_hole circle (at 1.27 -1.27) (size 1.524 1.524) (drill 1.016) (layers *.Cu *.Mask B.SilkS) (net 49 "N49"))
  (pad 6 thru_hole circle (at 1.27 1.27) (size 1.524 1.524) (drill 1.016) (layers *.Cu *.Mask B.SilkS) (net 1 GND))
  (pad 7 thru_hole circle (at 3.81 -1.27) (size 1.524 1.524) (drill 1.016) (layers *.Cu *.Mask B.SilkS) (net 16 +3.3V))
  (pad 8 thru_hole circle (at 3.81 1.27) (size 1.524 1.524) (drill 1.016) (layers *.Cu *.Mask B.SilkS) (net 16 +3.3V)))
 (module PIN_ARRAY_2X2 (layer F.Cu) (at 66.1 42.2)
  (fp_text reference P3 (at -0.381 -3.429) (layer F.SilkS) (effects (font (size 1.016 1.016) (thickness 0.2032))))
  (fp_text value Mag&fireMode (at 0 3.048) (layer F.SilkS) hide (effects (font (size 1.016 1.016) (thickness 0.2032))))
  (pad 1 thru_hole rect (at -1.27 1.27) (size 1.524 1.524) (drill 1.016) (layers *.Cu *.Mask F.SilkS) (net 51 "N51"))
  (pad 2 thru_hole circle (at -1.27 -1.27) (size 1.524 1.524) (drill 1.016) (layers *.Cu *.Mask F.SilkS) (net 52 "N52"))
  (pad 3 thru_hole circle (at 1.27 1.27) (size 1.524 1.524) (drill 1.016) (layers *.Cu *.Mask F.SilkS) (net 53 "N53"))
  (pad 4 thru_hole circle (at 1.27 -1.27) (size 1.524 1.524) (drill 1.016) (layers *.Cu *.Mask F.SilkS) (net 54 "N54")))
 (gr_line (start 111.6 71.9) (end 62.5 71.9) (angle 90) (layer Edge.Cuts) (width 0.15))
 (segment (start 91.425 61.275) (end 91.425 60.875) (width 0.254) (layer F.Cu) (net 19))
 (segment (start 91.425 60.875) (end 92.1 60.2) (width 0.254) (layer F.Cu) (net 19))
 (segment (start 92.1 60.2) (end 92.7 60.2) (width 0.254) (layer F.Cu) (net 19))
 (segment (start 92.7 60.2) (end 92.9 60) (width 0.254) (layer F.Cu) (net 19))
 (segment (start 92.9 60) (end 92.9 59) (width 0.254) (layer F.Cu) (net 19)) (via (at 92.9 59) (size 0.6) (layers F.Cu B.Cu) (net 19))
 (segment (start 92.9 59) (end 93.8525 59) (width 0.254) (layer B.Cu) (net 19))
 (segment (start 88.5475 57.1) (end 88.5475 59) (width 0.254) (layer B.Cu) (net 24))
 (segment (start 91.425 54.925) (end 91.425 55.225) (width 0.254) (layer F.Cu) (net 21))
 (segment (start 92.7 55.9) (end 92.9 56.1) (width 0.254) (layer F.Cu) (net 21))
 (segment (start 92.9 56.1) (end 92.9 57.1) (width 0.254) (layer F.Cu) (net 21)) (via (at 92.9 57.1) (size 0.6) (layers F.Cu B.Cu) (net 21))
 (segment (start 92.9 57.1) (end 93.8525 57.1) (width 0.254) (layer B.Cu) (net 21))
 (segment (start 91.425 55.225) (end 92.1 55.9) (width 0.254) (layer F.Cu) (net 21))
 (segment (start 92.1 55.9) (end 92.7 55.9) (width 0.254) (layer F.Cu) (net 21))
 (segment (start 91.9475 57.1) (end 90.4525 57.1) (width 0.254) (layer B.Cu) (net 28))
 (segment (start 70.6 70.5) (end 69 70.5) (width 0.254) (layer F.Cu) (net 55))
 (segment (start 65.44 64.2) (end 66.77 62.87) (width 0.254) (layer F.Cu) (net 55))
 (segment (start 63.6 64.2) (end 65.44 64.2) (width 0.254) (layer F.Cu) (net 55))
 (segment (start 63 64.8) (end 63.6 64.2) (width 0.254) (layer F.Cu) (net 55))
 (segment (start 63 68.7) (end 63 64.8) (width 0.254) (layer F.Cu) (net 55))
 (segment (start 63.5 69.2) (end 63 68.7) (width 0.254) (layer F.Cu) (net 55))
 (segment (start 67.7 69.2) (end 63.5 69.2) (width 0.254) (layer F.Cu) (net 55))
 (segment (start 69 70.5) (end 67.7 69.2) (width 0.254) (layer F.Cu) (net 55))
 (segment (start 90.4525 59) (end 91.9475 59) (width 0.254) (layer B.Cu) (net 27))
 (segment (start 64.23 70.49) (end 64.23 70.53) (width 0.254) (layer F.Cu) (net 57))
 (segment (start 73.5 71.6) (end 74.6 70.5) (width 0.254) (layer F.Cu) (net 57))
 (segment (start 65.3 71.6) (end 73.5 71.6) (width 0.254) (layer F.Cu) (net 57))
 (segment (start 64.23 70.53) (end 65.3 71.6) (width 0.254) (layer F.Cu) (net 57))
 (segment (start 66.77 67.95) (end 71.15 67.95) (width 0.254) (layer F.Cu) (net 56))
 (segment (start 72.6 69.4) (end 72.6 70.5) (width 0.254) (layer F.Cu) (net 56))
 (segment (start 71.15 67.95) (end 72.6 69.4) (width 0.254) (layer F.Cu) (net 56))
 (segment (start 66.77 70.49) (end 67.783 70.49) (width 0.254) (layer B.Cu) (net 14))
 (segment (start 67.783 70.49) (end 69.584 68.689) (width 0.254) (layer B.Cu) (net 14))
 (segment (start 64.23 67.95) (end 64.25 67.95) (width 0.254) (layer B.Cu) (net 2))
 (segment (start 72.495 64.4) (end 73.411 63.484) (width 0.254) (layer B.Cu) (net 2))
 (segment (start 69.1 64.4) (end 72.495 64.4) (width 0.254) (layer B.Cu) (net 2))
 (segment (start 68.5 65) (end 69.1 64.4) (width 0.254) (layer B.Cu) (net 2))
 (segment (start 68.5 65.6) (end 68.5 65) (width 0.254) (layer B.Cu) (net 2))
 (segment (start 67.4 66.7) (end 68.5 65.6) (width 0.254) (layer B.Cu) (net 2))
 (segment (start 65.5 66.7) (end 67.4 66.7) (width 0.254) (layer B.Cu) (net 2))
 (segment (start 64.25 67.95) (end 65.5 66.7) (width 0.254) (layer B.Cu) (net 2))
 (segment (start 66.77 65.41) (end 66.814002 65.41) (width 0.254) (layer F.Cu) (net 4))
 (segment (start 74.389 68.789) (end 73.384 68.789) (width 0.254) (layer B.Cu) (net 4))
 (segment (start 74.6 69) (end 74.389 68.789) (width 0.254) (layer B.Cu) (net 4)) (via (at 74.6 69) (size 0.6) (layers F.Cu B.Cu) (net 4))
 (segment (start 73.095998 67.495998) (end 74.6 69) (width 0.254) (layer F.Cu) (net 4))
 (segment (start 68.9 67.495998) (end 73.095998 67.495998) (width 0.254) (layer F.Cu) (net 4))
 (segment (start 66.814002 65.41) (end 68.9 67.495998) (width 0.254) (layer F.Cu) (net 4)))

